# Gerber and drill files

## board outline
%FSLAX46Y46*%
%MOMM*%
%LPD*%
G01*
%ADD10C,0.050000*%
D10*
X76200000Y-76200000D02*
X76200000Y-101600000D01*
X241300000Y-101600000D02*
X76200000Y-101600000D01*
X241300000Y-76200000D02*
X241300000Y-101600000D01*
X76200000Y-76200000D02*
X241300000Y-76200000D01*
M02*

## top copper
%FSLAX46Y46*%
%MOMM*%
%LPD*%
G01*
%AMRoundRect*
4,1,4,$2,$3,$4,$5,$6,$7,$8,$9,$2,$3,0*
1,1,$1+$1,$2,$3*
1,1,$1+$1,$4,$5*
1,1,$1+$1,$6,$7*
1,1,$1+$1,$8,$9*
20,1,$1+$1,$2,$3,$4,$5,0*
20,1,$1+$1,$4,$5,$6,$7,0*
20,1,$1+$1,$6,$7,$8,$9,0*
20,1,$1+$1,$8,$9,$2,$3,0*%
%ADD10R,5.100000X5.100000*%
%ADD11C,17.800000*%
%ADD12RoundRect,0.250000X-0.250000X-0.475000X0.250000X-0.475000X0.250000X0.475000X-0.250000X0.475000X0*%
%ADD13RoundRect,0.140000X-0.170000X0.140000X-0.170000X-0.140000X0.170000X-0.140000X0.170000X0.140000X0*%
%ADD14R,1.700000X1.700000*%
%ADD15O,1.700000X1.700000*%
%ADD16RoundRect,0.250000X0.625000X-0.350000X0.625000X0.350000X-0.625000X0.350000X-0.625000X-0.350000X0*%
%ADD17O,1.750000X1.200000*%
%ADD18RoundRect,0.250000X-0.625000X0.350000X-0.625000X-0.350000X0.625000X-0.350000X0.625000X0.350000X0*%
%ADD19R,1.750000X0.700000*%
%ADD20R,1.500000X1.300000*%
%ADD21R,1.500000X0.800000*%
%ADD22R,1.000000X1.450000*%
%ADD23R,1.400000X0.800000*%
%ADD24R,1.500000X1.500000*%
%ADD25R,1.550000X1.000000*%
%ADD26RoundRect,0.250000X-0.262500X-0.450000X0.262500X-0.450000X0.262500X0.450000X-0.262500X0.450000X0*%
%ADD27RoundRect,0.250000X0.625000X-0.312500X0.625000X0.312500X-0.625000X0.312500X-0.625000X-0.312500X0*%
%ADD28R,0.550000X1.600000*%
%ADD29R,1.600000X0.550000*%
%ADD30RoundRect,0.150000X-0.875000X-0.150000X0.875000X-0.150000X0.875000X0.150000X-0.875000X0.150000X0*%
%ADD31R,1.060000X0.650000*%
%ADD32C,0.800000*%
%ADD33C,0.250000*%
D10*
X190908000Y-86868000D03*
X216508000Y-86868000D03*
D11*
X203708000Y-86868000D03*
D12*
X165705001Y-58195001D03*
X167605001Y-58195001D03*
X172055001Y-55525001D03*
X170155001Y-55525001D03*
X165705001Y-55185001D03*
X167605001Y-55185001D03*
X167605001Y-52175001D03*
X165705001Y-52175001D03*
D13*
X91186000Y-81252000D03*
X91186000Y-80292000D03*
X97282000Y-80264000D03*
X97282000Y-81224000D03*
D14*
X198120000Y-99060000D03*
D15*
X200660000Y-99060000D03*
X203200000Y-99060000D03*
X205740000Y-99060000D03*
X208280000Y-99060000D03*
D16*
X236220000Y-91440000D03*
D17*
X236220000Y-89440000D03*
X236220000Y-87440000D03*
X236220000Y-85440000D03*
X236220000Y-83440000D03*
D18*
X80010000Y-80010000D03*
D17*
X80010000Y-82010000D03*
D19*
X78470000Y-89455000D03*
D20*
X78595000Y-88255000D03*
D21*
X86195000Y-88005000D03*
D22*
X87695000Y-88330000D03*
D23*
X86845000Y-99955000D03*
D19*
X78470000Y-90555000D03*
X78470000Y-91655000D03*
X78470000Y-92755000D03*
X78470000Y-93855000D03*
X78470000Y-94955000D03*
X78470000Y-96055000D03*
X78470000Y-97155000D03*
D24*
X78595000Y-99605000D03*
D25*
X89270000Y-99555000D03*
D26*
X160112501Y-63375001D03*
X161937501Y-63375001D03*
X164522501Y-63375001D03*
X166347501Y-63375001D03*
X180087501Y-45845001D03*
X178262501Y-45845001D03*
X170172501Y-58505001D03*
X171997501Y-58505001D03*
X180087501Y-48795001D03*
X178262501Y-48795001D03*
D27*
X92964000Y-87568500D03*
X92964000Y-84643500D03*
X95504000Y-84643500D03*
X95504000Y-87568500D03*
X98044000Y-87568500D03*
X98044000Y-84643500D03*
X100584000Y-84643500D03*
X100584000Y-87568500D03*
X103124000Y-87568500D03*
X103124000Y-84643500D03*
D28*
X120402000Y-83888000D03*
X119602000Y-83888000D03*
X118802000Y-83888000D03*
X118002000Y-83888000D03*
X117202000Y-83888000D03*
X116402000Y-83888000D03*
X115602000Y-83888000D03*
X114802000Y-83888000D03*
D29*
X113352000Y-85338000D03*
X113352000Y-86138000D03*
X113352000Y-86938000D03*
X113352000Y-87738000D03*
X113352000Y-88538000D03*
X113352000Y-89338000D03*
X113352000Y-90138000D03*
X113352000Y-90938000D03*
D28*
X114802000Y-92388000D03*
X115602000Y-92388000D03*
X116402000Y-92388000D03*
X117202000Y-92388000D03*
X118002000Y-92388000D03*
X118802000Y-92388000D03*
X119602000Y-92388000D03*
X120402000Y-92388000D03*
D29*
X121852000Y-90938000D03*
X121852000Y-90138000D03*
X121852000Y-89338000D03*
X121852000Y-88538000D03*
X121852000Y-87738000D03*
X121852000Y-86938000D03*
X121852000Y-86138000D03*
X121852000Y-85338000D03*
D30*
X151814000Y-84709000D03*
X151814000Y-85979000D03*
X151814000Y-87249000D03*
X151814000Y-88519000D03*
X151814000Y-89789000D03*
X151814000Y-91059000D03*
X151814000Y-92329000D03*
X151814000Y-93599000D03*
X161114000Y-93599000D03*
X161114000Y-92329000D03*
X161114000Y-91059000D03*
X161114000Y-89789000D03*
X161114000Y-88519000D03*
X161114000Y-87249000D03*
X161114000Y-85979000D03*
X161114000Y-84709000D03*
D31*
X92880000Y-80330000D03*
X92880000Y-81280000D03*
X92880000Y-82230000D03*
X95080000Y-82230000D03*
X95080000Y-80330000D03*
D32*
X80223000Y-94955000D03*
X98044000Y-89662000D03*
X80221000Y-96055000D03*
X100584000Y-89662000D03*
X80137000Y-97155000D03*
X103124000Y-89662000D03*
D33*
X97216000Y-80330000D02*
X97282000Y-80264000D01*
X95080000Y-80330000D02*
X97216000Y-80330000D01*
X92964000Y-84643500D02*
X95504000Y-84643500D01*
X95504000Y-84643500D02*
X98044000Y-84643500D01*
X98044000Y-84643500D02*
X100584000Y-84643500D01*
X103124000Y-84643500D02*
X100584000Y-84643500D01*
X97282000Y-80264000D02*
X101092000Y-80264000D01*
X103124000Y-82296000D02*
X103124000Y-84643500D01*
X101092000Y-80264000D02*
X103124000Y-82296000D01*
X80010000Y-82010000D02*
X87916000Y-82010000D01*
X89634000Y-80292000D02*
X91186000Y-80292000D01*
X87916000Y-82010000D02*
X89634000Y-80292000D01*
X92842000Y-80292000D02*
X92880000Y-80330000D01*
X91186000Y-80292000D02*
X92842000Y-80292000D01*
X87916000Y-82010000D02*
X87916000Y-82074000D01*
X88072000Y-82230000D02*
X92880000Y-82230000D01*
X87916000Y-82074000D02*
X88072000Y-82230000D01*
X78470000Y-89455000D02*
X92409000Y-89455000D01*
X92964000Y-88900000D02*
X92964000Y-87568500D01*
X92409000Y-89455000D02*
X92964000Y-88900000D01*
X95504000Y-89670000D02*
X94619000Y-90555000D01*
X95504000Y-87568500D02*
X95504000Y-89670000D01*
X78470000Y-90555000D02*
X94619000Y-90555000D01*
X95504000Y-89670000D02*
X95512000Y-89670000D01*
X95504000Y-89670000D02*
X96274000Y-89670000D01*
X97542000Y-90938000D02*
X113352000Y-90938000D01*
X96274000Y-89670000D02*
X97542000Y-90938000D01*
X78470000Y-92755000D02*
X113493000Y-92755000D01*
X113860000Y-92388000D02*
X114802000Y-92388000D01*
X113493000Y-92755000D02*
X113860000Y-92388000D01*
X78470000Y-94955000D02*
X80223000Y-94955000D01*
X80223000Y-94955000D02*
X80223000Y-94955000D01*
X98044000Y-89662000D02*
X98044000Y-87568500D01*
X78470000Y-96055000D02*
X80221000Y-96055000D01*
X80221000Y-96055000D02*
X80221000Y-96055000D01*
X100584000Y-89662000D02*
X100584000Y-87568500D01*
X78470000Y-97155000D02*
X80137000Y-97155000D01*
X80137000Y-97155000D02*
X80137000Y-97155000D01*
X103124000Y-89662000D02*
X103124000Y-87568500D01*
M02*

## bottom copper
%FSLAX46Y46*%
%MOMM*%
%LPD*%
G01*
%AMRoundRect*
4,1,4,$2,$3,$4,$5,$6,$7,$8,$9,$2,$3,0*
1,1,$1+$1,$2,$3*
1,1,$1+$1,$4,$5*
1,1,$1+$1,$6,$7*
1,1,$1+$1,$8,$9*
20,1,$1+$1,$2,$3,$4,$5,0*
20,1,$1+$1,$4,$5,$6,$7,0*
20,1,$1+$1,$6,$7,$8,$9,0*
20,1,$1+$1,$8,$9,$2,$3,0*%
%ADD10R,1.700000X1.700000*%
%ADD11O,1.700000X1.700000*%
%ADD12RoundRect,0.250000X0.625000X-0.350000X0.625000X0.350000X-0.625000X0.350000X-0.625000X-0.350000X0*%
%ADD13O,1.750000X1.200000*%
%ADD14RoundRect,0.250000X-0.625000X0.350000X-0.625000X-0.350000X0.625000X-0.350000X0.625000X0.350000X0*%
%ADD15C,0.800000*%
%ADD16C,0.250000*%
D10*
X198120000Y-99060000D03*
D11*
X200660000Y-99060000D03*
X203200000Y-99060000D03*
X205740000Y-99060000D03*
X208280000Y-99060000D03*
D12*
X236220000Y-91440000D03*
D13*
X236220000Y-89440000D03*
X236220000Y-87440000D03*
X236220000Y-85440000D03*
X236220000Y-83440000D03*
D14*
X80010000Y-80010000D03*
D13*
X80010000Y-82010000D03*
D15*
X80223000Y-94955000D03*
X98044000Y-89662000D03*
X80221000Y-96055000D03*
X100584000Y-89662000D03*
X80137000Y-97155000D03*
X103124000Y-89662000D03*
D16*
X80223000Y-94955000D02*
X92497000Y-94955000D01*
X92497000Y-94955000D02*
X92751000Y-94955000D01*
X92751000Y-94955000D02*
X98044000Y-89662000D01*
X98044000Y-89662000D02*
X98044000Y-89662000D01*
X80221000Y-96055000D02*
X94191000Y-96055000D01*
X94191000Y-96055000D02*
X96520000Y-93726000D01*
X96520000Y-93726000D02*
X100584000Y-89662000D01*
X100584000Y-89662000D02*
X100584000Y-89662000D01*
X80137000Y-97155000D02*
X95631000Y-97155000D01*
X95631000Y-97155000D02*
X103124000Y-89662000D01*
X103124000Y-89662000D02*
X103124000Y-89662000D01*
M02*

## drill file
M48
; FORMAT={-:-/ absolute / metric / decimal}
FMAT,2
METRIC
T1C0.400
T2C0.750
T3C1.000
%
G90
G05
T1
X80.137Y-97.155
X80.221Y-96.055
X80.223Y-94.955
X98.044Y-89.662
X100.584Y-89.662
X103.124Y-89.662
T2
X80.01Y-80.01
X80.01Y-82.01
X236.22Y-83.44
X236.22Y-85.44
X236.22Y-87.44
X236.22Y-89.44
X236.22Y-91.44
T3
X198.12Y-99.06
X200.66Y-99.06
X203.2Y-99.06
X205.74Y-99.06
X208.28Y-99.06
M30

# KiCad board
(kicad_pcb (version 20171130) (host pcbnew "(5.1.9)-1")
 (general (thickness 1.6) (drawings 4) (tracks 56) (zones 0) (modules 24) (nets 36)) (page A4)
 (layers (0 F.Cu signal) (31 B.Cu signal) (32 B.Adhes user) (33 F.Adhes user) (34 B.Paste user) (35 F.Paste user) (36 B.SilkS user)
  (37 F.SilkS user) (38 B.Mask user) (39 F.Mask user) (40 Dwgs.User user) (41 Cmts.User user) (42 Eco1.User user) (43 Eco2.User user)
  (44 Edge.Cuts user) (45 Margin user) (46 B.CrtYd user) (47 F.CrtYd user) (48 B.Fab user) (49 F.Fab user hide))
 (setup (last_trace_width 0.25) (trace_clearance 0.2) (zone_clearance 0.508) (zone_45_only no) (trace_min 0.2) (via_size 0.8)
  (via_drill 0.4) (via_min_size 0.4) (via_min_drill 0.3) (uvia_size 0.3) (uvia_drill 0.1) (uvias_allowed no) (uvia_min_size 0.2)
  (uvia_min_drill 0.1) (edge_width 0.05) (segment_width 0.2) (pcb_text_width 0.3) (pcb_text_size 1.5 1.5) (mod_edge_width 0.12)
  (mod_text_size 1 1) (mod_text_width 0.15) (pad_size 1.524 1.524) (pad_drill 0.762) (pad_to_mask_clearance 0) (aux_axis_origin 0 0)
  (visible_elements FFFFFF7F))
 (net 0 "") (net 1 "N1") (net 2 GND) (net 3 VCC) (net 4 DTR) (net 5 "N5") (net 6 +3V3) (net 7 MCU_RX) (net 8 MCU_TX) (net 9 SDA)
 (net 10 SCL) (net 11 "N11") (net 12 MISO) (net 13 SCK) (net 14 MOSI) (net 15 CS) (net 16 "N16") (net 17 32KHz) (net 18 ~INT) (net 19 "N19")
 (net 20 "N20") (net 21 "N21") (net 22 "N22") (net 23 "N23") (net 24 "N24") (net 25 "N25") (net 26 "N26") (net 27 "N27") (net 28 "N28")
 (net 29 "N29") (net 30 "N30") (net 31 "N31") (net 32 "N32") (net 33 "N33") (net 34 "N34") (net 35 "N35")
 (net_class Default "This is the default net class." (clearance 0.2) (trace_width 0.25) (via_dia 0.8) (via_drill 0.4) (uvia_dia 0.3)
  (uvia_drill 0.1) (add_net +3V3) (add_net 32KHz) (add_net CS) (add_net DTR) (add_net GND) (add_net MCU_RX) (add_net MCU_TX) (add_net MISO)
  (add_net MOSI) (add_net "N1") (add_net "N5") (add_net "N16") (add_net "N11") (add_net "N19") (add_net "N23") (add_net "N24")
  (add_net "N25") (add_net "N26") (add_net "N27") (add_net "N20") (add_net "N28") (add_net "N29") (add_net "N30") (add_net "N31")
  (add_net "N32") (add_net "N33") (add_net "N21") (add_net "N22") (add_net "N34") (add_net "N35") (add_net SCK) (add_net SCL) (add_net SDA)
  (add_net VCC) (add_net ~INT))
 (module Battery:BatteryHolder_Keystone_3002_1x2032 (layer F.Cu) (at 203.708 86.868 180)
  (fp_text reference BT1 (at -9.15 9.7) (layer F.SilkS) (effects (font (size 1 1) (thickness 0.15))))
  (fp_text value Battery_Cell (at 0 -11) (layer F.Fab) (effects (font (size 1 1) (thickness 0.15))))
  (pad 1 smd rect (at 12.8 0 180) (size 5.1 5.1) (layers F.Cu F.Paste F.Mask) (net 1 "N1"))
  (pad 1 smd rect (at -12.8 0 180) (size 5.1 5.1) (layers F.Cu F.Paste F.Mask) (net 1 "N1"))
  (pad 2 smd circle (at 0 0 180) (size 17.8 17.8) (layers F.Cu F.Mask) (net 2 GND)))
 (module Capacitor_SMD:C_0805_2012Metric (layer F.Cu) (at 166.655001 58.195001)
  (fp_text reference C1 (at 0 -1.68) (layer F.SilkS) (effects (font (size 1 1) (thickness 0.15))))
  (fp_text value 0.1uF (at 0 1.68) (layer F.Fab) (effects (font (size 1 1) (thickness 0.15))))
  (pad 1 smd roundrect (at -0.95 0) (size 1 1.45) (layers F.Cu F.Paste F.Mask) (roundrect_rratio 0.25) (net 2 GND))
  (pad 2 smd roundrect (at 0.95 0) (size 1 1.45) (layers F.Cu F.Paste F.Mask) (roundrect_rratio 0.25) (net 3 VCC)))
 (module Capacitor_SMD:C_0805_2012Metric (layer F.Cu) (at 171.105001 55.525001)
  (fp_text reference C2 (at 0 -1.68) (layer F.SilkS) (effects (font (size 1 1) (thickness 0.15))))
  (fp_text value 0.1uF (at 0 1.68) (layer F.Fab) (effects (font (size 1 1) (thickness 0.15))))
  (pad 2 smd roundrect (at 0.95 0) (size 1 1.45) (layers F.Cu F.Paste F.Mask) (roundrect_rratio 0.25) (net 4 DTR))
  (pad 1 smd roundrect (at -0.95 0) (size 1 1.45) (layers F.Cu F.Paste F.Mask) (roundrect_rratio 0.25) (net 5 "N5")))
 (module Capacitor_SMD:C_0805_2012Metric (layer F.Cu) (at 166.655001 55.185001)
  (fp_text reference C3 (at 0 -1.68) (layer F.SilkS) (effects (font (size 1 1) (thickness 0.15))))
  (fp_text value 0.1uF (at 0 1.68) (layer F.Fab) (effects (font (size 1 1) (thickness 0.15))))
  (pad 1 smd roundrect (at -0.95 0) (size 1 1.45) (layers F.Cu F.Paste F.Mask) (roundrect_rratio 0.25) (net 3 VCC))
  (pad 2 smd roundrect (at 0.95 0) (size 1 1.45) (layers F.Cu F.Paste F.Mask) (roundrect_rratio 0.25) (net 2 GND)))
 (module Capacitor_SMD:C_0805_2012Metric (layer F.Cu) (at 166.655001 52.175001)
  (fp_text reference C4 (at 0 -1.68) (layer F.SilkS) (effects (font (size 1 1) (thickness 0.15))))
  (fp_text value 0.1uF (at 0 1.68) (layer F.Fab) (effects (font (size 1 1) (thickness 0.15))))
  (pad 2 smd roundrect (at 0.95 0) (size 1 1.45) (layers F.Cu F.Paste F.Mask) (roundrect_rratio 0.25) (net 2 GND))
  (pad 1 smd roundrect (at -0.95 0) (size 1 1.45) (layers F.Cu F.Paste F.Mask) (roundrect_rratio 0.25) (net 3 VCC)))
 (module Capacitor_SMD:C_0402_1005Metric (layer F.Cu) (at 91.186 80.772 270)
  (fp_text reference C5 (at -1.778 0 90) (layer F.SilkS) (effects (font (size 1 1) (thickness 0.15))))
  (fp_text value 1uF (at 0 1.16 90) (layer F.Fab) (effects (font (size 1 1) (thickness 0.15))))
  (pad 2 smd roundrect (at 0.48 0 270) (size 0.56 0.62) (layers F.Cu F.Paste F.Mask) (roundrect_rratio 0.25) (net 2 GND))
  (pad 1 smd roundrect (at -0.48 0 270) (size 0.56 0.62) (layers F.Cu F.Paste F.Mask) (roundrect_rratio 0.25) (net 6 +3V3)))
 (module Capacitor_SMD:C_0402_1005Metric (layer F.Cu) (at 97.282 80.744 270)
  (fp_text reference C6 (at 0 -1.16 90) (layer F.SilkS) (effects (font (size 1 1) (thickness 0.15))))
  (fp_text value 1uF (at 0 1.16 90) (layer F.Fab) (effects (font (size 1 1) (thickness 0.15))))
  (pad 1 smd roundrect (at -0.48 0 270) (size 0.56 0.62) (layers F.Cu F.Paste F.Mask) (roundrect_rratio 0.25) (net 3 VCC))
  (pad 2 smd roundrect (at 0.48 0 270) (size 0.56 0.62) (layers F.Cu F.Paste F.Mask) (roundrect_rratio 0.25) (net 2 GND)))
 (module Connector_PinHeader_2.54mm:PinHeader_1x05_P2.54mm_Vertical (layer F.Cu) (at 198.12 99.06 90)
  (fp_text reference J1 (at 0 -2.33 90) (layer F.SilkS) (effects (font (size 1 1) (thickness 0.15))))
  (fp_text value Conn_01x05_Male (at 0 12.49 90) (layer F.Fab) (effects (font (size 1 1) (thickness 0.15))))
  (pad 1 thru_hole rect (at 0 0 90) (size 1.7 1.7) (drill 1) (layers *.Cu *.Mask) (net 2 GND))
  (pad 2 thru_hole oval (at 0 2.54 90) (size 1.7 1.7) (drill 1) (layers *.Cu *.Mask) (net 3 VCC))
  (pad 3 thru_hole oval (at 0 5.08 90) (size 1.7 1.7) (drill 1) (layers *.Cu *.Mask) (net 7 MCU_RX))
  (pad 4 thru_hole oval (at 0 7.62 90) (size 1.7 1.7) (drill 1) (layers *.Cu *.Mask) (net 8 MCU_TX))
  (pad 5 thru_hole oval (at 0 10.16 90) (size 1.7 1.7) (drill 1) (layers *.Cu *.Mask) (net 5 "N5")))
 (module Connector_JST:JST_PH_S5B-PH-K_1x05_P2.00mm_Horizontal (layer F.Cu) (at 236.22 91.44 90)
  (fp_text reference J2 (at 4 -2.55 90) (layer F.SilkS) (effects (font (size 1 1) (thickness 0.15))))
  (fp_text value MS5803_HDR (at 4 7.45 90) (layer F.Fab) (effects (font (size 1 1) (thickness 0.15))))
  (pad 1 thru_hole roundrect (at 0 0 90) (size 1.2 1.75) (drill 0.75) (layers *.Cu *.Mask) (roundrect_rratio 0.208333) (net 2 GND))
  (pad 2 thru_hole oval (at 2 0 90) (size 1.2 1.75) (drill 0.75) (layers *.Cu *.Mask) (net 3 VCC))
  (pad 3 thru_hole oval (at 4 0 90) (size 1.2 1.75) (drill 0.75) (layers *.Cu *.Mask) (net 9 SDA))
  (pad 4 thru_hole oval (at 6 0 90) (size 1.2 1.75) (drill 0.75) (layers *.Cu *.Mask) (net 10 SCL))
  (pad 5 thru_hole oval (at 8 0 90) (size 1.2 1.75) (drill 0.75) (layers *.Cu *.Mask)))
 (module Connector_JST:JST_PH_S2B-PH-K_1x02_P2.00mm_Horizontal (layer F.Cu) (at 80.01 80.01 270)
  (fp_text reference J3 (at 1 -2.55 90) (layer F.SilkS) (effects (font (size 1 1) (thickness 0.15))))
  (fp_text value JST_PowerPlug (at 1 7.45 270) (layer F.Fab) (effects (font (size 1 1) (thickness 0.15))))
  (pad 1 thru_hole roundrect (at 0 0 270) (size 1.2 1.75) (drill 0.75) (layers *.Cu *.Mask) (roundrect_rratio 0.208333) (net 2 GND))
  (pad 2 thru_hole oval (at 2 0 270) (size 1.2 1.75) (drill 0.75) (layers *.Cu *.Mask) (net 6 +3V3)))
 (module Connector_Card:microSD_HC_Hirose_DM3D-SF (layer F.Cu) (at 83.82 93.98 270)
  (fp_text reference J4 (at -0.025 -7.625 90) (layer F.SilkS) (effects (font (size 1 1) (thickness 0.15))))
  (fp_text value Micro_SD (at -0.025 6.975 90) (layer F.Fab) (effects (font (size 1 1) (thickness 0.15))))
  (pad 8 smd rect (at -4.525 5.35 270) (size 0.7 1.75) (layers F.Cu F.Paste F.Mask) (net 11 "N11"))
  (pad 11 smd rect (at -5.725 5.225 270) (size 1.3 1.5) (layers F.Cu F.Paste F.Mask))
  (pad 11 smd rect (at -5.975 -2.375 270) (size 0.8 1.5) (layers F.Cu F.Paste F.Mask))
  (pad 9 smd rect (at -5.65 -3.875 270) (size 1.45 1) (layers F.Cu F.Paste F.Mask) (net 2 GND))
  (pad 11 smd rect (at 5.975 -3.025 270) (size 0.8 1.4) (layers F.Cu F.Paste F.Mask))
  (pad 7 smd rect (at -3.425 5.35 270) (size 0.7 1.75) (layers F.Cu F.Paste F.Mask) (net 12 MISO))
  (pad 6 smd rect (at -2.325 5.35 270) (size 0.7 1.75) (layers F.Cu F.Paste F.Mask) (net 2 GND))
  (pad 5 smd rect (at -1.225 5.35 270) (size 0.7 1.75) (layers F.Cu F.Paste F.Mask) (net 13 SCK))
  (pad 4 smd rect (at -0.125 5.35 270) (size 0.7 1.75) (layers F.Cu F.Paste F.Mask) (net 3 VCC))
  (pad 3 smd rect (at 0.975 5.35 270) (size 0.7 1.75) (layers F.Cu F.Paste F.Mask) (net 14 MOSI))
  (pad 2 smd rect (at 2.075 5.35 270) (size 0.7 1.75) (layers F.Cu F.Paste F.Mask) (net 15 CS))
  (pad 1 smd rect (at 3.175 5.35 270) (size 0.7 1.75) (layers F.Cu F.Paste F.Mask) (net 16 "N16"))
  (pad 11 smd rect (at 5.625 5.225 270) (size 1.5 1.5) (layers F.Cu F.Paste F.Mask))
  (pad 10 smd rect (at 5.575 -5.45 270) (size 1 1.55) (layers F.Cu F.Paste F.Mask)))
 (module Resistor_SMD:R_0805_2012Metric (layer F.Cu) (at 161.025001 63.375001)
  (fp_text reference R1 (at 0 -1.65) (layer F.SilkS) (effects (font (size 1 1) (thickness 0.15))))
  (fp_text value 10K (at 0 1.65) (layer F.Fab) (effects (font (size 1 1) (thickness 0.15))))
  (pad 1 smd roundrect (at -0.9125 0) (size 1.025 1.4) (layers F.Cu F.Paste F.Mask) (roundrect_rratio 0.243902) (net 3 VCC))
  (pad 2 smd roundrect (at 0.9125 0) (size 1.025 1.4) (layers F.Cu F.Paste F.Mask) (roundrect_rratio 0.243902) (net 4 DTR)))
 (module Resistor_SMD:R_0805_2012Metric (layer F.Cu) (at 165.435001 63.375001)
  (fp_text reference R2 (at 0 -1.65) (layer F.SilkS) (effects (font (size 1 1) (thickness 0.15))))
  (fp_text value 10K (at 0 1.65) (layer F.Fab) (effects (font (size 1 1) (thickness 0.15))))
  (pad 1 smd roundrect (at -0.9125 0) (size 1.025 1.4) (layers F.Cu F.Paste F.Mask) (roundrect_rratio 0.243902) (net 3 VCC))
  (pad 2 smd roundrect (at 0.9125 0) (size 1.025 1.4) (layers F.Cu F.Paste F.Mask) (roundrect_rratio 0.243902) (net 10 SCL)))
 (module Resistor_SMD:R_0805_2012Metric (layer F.Cu) (at 179.175001 45.845001)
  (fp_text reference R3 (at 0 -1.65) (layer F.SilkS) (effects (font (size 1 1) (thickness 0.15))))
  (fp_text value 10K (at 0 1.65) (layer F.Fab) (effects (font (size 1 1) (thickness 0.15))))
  (pad 2 smd roundrect (at 0.9125 0) (size 1.025 1.4) (layers F.Cu F.Paste F.Mask) (roundrect_rratio 0.243902) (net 9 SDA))
  (pad 1 smd roundrect (at -0.9125 0) (size 1.025 1.4) (layers F.Cu F.Paste F.Mask) (roundrect_rratio 0.243902) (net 3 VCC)))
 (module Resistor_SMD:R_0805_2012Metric (layer F.Cu) (at 171.085001 58.505001)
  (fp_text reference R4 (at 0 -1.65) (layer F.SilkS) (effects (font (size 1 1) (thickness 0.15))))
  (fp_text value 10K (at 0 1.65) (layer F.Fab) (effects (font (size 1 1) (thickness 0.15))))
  (pad 1 smd roundrect (at -0.9125 0) (size 1.025 1.4) (layers F.Cu F.Paste F.Mask) (roundrect_rratio 0.243902) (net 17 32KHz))
  (pad 2 smd roundrect (at 0.9125 0) (size 1.025 1.4) (layers F.Cu F.Paste F.Mask) (roundrect_rratio 0.243902) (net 3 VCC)))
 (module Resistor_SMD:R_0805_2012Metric (layer F.Cu) (at 179.175001 48.795001)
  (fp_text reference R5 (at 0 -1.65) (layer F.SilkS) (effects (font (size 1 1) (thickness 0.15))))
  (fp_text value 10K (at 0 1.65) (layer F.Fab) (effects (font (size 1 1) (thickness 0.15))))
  (pad 2 smd roundrect (at 0.9125 0) (size 1.025 1.4) (layers F.Cu F.Paste F.Mask) (roundrect_rratio 0.243902) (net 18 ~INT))
  (pad 1 smd roundrect (at -0.9125 0) (size 1.025 1.4) (layers F.Cu F.Paste F.Mask) (roundrect_rratio 0.243902) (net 3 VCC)))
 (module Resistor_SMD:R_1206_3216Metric (layer F.Cu) (at 92.964 86.106 90)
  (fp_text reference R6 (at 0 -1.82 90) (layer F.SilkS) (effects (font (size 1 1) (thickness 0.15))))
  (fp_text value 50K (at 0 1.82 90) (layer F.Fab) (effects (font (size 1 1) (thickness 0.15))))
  (pad 1 smd roundrect (at -1.4625 0 90) (size 1.125 1.75) (layers F.Cu F.Paste F.Mask) (roundrect_rratio 0.222222) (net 11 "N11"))
  (pad 2 smd roundrect (at 1.4625 0 90) (size 1.125 1.75) (layers F.Cu F.Paste F.Mask) (roundrect_rratio 0.222222) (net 3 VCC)))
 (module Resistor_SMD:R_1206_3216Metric (layer F.Cu) (at 95.504 86.106 90)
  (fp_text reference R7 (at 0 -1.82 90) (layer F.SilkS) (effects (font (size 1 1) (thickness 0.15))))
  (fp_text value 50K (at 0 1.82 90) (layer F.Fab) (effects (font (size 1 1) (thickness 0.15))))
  (pad 2 smd roundrect (at 1.4625 0 90) (size 1.125 1.75) (layers F.Cu F.Paste F.Mask) (roundrect_rratio 0.222222) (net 3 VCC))
  (pad 1 smd roundrect (at -1.4625 0 90) (size 1.125 1.75) (layers F.Cu F.Paste F.Mask) (roundrect_rratio 0.222222) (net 12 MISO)))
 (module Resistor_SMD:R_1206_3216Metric (layer F.Cu) (at 98.044 86.106 90)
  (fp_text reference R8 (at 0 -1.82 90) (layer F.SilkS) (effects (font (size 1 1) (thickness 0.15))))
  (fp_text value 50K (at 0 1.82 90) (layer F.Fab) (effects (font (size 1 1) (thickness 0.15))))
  (pad 1 smd roundrect (at -1.4625 0 90) (size 1.125 1.75) (layers F.Cu F.Paste F.Mask) (roundrect_rratio 0.222222) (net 14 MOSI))
  (pad 2 smd roundrect (at 1.4625 0 90) (size 1.125 1.75) (layers F.Cu F.Paste F.Mask) (roundrect_rratio 0.222222) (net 3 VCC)))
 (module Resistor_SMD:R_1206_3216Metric (layer F.Cu) (at 100.584 86.106 90)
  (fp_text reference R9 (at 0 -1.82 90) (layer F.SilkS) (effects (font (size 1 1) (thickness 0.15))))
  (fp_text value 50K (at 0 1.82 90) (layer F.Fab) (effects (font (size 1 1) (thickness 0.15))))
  (pad 2 smd roundrect (at 1.4625 0 90) (size 1.125 1.75) (layers F.Cu F.Paste F.Mask) (roundrect_rratio 0.222222) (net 3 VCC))
  (pad 1 smd roundrect (at -1.4625 0 90) (size 1.125 1.75) (layers F.Cu F.Paste F.Mask) (roundrect_rratio 0.222222) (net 15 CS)))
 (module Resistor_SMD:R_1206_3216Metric (layer F.Cu) (at 103.124 86.106 90)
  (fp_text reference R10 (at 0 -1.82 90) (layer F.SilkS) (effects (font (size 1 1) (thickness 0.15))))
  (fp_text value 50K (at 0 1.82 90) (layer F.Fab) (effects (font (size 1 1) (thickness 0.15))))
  (pad 1 smd roundrect (at -1.4625 0 90) (size 1.125 1.75) (layers F.Cu F.Paste F.Mask) (roundrect_rratio 0.222222) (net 16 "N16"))
  (pad 2 smd roundrect (at 1.4625 0 90) (size 1.125 1.75) (layers F.Cu F.Paste F.Mask) (roundrect_rratio 0.222222) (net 3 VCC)))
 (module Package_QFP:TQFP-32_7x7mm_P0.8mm (layer F.Cu) (at 117.602 88.138 270)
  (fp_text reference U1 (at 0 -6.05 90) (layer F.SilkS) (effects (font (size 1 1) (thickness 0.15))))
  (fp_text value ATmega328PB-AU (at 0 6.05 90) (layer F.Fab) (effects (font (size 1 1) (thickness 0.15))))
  (pad 1 smd rect (at -4.25 -2.8 270) (size 1.6 0.55) (layers F.Cu F.Paste F.Mask) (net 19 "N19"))
  (pad 2 smd rect (at -4.25 -2 270) (size 1.6 0.55) (layers F.Cu F.Paste F.Mask) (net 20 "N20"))
  (pad 3 smd rect (at -4.25 -1.2 270) (size 1.6 0.55) (layers F.Cu F.Paste F.Mask) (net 2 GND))
  (pad 4 smd rect (at -4.25 -0.4 270) (size 1.6 0.55) (layers F.Cu F.Paste F.Mask) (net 3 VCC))
  (pad 5 smd rect (at -4.25 0.4 270) (size 1.6 0.55) (layers F.Cu F.Paste F.Mask) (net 2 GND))
  (pad 6 smd rect (at -4.25 1.2 270) (size 1.6 0.55) (layers F.Cu F.Paste F.Mask) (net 3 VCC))
  (pad 7 smd rect (at -4.25 2 270) (size 1.6 0.55) (layers F.Cu F.Paste F.Mask) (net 17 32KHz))
  (pad 8 smd rect (at -4.25 2.8 270) (size 1.6 0.55) (layers F.Cu F.Paste F.Mask) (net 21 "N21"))
  (pad 9 smd rect (at -2.8 4.25) (size 1.6 0.55) (layers F.Cu F.Paste F.Mask) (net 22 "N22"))
  (pad 10 smd rect (at -2 4.25) (size 1.6 0.55) (layers F.Cu F.Paste F.Mask) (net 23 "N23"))
  (pad 11 smd rect (at -1.2 4.25) (size 1.6 0.55) (layers F.Cu F.Paste F.Mask) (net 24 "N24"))
  (pad 12 smd rect (at -0.4 4.25) (size 1.6 0.55) (layers F.Cu F.Paste F.Mask) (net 15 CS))
  (pad 13 smd rect (at 0.4 4.25) (size 1.6 0.55) (layers F.Cu F.Paste F.Mask) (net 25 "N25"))
  (pad 14 smd rect (at 1.2 4.25) (size 1.6 0.55) (layers F.Cu F.Paste F.Mask) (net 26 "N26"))
  (pad 15 smd rect (at 2 4.25) (size 1.6 0.55) (layers F.Cu F.Paste F.Mask) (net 14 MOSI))
  (pad 16 smd rect (at 2.8 4.25) (size 1.6 0.55) (layers F.Cu F.Paste F.Mask) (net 12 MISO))
  (pad 17 smd rect (at 4.25 2.8 270) (size 1.6 0.55) (layers F.Cu F.Paste F.Mask) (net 13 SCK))
  (pad 18 smd rect (at 4.25 2 270) (size 1.6 0.55) (layers F.Cu F.Paste F.Mask) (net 3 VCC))
  (pad 19 smd rect (at 4.25 1.2 270) (size 1.6 0.55) (layers F.Cu F.Paste F.Mask) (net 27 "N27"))
  (pad 20 smd rect (at 4.25 0.4 270) (size 1.6 0.55) (layers F.Cu F.Paste F.Mask) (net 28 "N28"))
  (pad 21 smd rect (at 4.25 -0.4 270) (size 1.6 0.55) (layers F.Cu F.Paste F.Mask) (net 2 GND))
  (pad 22 smd rect (at 4.25 -1.2 270) (size 1.6 0.55) (layers F.Cu F.Paste F.Mask) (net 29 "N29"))
  (pad 23 smd rect (at 4.25 -2 270) (size 1.6 0.55) (layers F.Cu F.Paste F.Mask) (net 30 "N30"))
  (pad 24 smd rect (at 4.25 -2.8 270) (size 1.6 0.55) (layers F.Cu F.Paste F.Mask) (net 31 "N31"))
  (pad 25 smd rect (at 2.8 -4.25) (size 1.6 0.55) (layers F.Cu F.Paste F.Mask) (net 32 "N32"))
  (pad 26 smd rect (at 2 -4.25) (size 1.6 0.55) (layers F.Cu F.Paste F.Mask) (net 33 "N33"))
  (pad 27 smd rect (at 1.2 -4.25) (size 1.6 0.55) (layers F.Cu F.Paste F.Mask) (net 9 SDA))
  (pad 28 smd rect (at 0.4 -4.25) (size 1.6 0.55) (layers F.Cu F.Paste F.Mask) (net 10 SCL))
  (pad 29 smd rect (at -0.4 -4.25) (size 1.6 0.55) (layers F.Cu F.Paste F.Mask) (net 4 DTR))
  (pad 30 smd rect (at -1.2 -4.25) (size 1.6 0.55) (layers F.Cu F.Paste F.Mask) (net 7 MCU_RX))
  (pad 31 smd rect (at -2 -4.25) (size 1.6 0.55) (layers F.Cu F.Paste F.Mask) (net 8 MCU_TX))
  (pad 32 smd rect (at -2.8 -4.25) (size 1.6 0.55) (layers F.Cu F.Paste F.Mask) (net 18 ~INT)))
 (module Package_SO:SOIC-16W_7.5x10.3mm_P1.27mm (layer F.Cu) (at 156.464 89.154)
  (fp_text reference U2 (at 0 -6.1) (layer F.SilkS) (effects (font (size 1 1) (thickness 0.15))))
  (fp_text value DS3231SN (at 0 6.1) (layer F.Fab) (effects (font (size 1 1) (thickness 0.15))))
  (pad 1 smd roundrect (at -4.65 -4.445) (size 2.05 0.6) (layers F.Cu F.Paste F.Mask) (roundrect_rratio 0.25) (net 17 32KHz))
  (pad 2 smd roundrect (at -4.65 -3.175) (size 2.05 0.6) (layers F.Cu F.Paste F.Mask) (roundrect_rratio 0.25) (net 3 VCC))
  (pad 3 smd roundrect (at -4.65 -1.905) (size 2.05 0.6) (layers F.Cu F.Paste F.Mask) (roundrect_rratio 0.25) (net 18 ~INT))
  (pad 4 smd roundrect (at -4.65 -0.635) (size 2.05 0.6) (layers F.Cu F.Paste F.Mask) (roundrect_rratio 0.25) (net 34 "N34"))
  (pad 5 smd roundrect (at -4.65 0.635) (size 2.05 0.6) (layers F.Cu F.Paste F.Mask) (roundrect_rratio 0.25) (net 2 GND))
  (pad 6 smd roundrect (at -4.65 1.905) (size 2.05 0.6) (layers F.Cu F.Paste F.Mask) (roundrect_rratio 0.25) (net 2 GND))
  (pad 7 smd roundrect (at -4.65 3.175) (size 2.05 0.6) (layers F.Cu F.Paste F.Mask) (roundrect_rratio 0.25) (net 2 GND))
  (pad 8 smd roundrect (at -4.65 4.445) (size 2.05 0.6) (layers F.Cu F.Paste F.Mask) (roundrect_rratio 0.25) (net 2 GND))
  (pad 9 smd roundrect (at 4.65 4.445) (size 2.05 0.6) (layers F.Cu F.Paste F.Mask) (roundrect_rratio 0.25) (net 2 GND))
  (pad 10 smd roundrect (at 4.65 3.175) (size 2.05 0.6) (layers F.Cu F.Paste F.Mask) (roundrect_rratio 0.25) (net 2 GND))
  (pad 11 smd roundrect (at 4.65 1.905) (size 2.05 0.6) (layers F.Cu F.Paste F.Mask) (roundrect_rratio 0.25) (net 2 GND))
  (pad 12 smd roundrect (at 4.65 0.635) (size 2.05 0.6) (layers F.Cu F.Paste F.Mask) (roundrect_rratio 0.25) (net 2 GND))
  (pad 13 smd roundrect (at 4.65 -0.635) (size 2.05 0.6) (layers F.Cu F.Paste F.Mask) (roundrect_rratio 0.25) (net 2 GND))
  (pad 14 smd roundrect (at 4.65 -1.905) (size 2.05 0.6) (layers F.Cu F.Paste F.Mask) (roundrect_rratio 0.25) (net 1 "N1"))
  (pad 15 smd roundrect (at 4.65 -3.175) (size 2.05 0.6) (layers F.Cu F.Paste F.Mask) (roundrect_rratio 0.25) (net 9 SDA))
  (pad 16 smd roundrect (at 4.65 -4.445) (size 2.05 0.6) (layers F.Cu F.Paste F.Mask) (roundrect_rratio 0.25) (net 10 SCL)))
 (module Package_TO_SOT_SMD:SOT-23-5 (layer F.Cu) (at 93.98 81.28)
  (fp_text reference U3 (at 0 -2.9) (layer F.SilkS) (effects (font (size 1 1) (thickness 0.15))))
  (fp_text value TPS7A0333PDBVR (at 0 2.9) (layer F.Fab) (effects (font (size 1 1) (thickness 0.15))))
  (pad 1 smd rect (at -1.1 -0.95) (size 1.06 0.65) (layers F.Cu F.Paste F.Mask) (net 6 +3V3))
  (pad 2 smd rect (at -1.1 0) (size 1.06 0.65) (layers F.Cu F.Paste F.Mask) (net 2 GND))
  (pad 3 smd rect (at -1.1 0.95) (size 1.06 0.65) (layers F.Cu F.Paste F.Mask) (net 6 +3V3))
  (pad 4 smd rect (at 1.1 0.95) (size 1.06 0.65) (layers F.Cu F.Paste F.Mask) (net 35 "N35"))
  (pad 5 smd rect (at 1.1 -0.95) (size 1.06 0.65) (layers F.Cu F.Paste F.Mask) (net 3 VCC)))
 (gr_line (start 76.2 76.2) (end 76.2 101.6) (layer Edge.Cuts) (width 0.05))
 (gr_line (start 241.3 101.6) (end 76.2 101.6) (layer Edge.Cuts) (width 0.05))
 (gr_line (start 241.3 76.2) (end 241.3 101.6) (layer Edge.Cuts) (width 0.05))
 (gr_line (start 76.2 76.2) (end 241.3 76.2) (layer Edge.Cuts) (width 0.05))
 (segment (start 97.216 80.33) (end 97.282 80.264) (width 0.25) (layer F.Cu) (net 3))
 (segment (start 95.08 80.33) (end 97.216 80.33) (width 0.25) (layer F.Cu) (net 3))
 (segment (start 92.964 84.6435) (end 95.504 84.6435) (width 0.25) (layer F.Cu) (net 3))
 (segment (start 95.504 84.6435) (end 98.044 84.6435) (width 0.25) (layer F.Cu) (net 3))
 (segment (start 98.044 84.6435) (end 100.584 84.6435) (width 0.25) (layer F.Cu) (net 3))
 (segment (start 103.124 84.6435) (end 100.584 84.6435) (width 0.25) (layer F.Cu) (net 3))
 (segment (start 97.282 80.264) (end 101.092 80.264) (width 0.25) (layer F.Cu) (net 3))
 (segment (start 103.124 82.296) (end 103.124 84.6435) (width 0.25) (layer F.Cu) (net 3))
 (segment (start 101.092 80.264) (end 103.124 82.296) (width 0.25) (layer F.Cu) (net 3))
 (segment (start 80.01 82.01) (end 87.916 82.01) (width 0.25) (layer F.Cu) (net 6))
 (segment (start 89.634 80.292) (end 91.186 80.292) (width 0.25) (layer F.Cu) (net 6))
 (segment (start 87.916 82.01) (end 89.634 80.292) (width 0.25) (layer F.Cu) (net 6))
 (segment (start 92.842 80.292) (end 92.88 80.33) (width 0.25) (layer F.Cu) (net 6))
 (segment (start 91.186 80.292) (end 92.842 80.292) (width 0.25) (layer F.Cu) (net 6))
 (segment (start 87.916 82.01) (end 87.916 82.074) (width 0.25) (layer F.Cu) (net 6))
 (segment (start 88.072 82.23) (end 92.88 82.23) (width 0.25) (layer F.Cu) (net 6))
 (segment (start 87.916 82.074) (end 88.072 82.23) (width 0.25) (layer F.Cu) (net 6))
 (segment (start 78.47 89.455) (end 92.409 89.455) (width 0.25) (layer F.Cu) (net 11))
 (segment (start 92.964 88.9) (end 92.964 87.5685) (width 0.25) (layer F.Cu) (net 11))
 (segment (start 92.409 89.455) (end 92.964 88.9) (width 0.25) (layer F.Cu) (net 11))
 (segment (start 95.504 89.67) (end 94.619 90.555) (width 0.25) (layer F.Cu) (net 12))
 (segment (start 95.504 87.5685) (end 95.504 89.67) (width 0.25) (layer F.Cu) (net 12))
 (segment (start 78.47 90.555) (end 94.619 90.555) (width 0.25) (layer F.Cu) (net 12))
 (segment (start 95.504 89.67) (end 95.512 89.67) (width 0.25) (layer F.Cu) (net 12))
 (segment (start 95.504 89.67) (end 96.274 89.67) (width 0.25) (layer F.Cu) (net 12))
 (segment (start 97.542 90.938) (end 113.352 90.938) (width 0.25) (layer F.Cu) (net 12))
 (segment (start 96.274 89.67) (end 97.542 90.938) (width 0.25) (layer F.Cu) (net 12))
 (segment (start 78.47 92.755) (end 113.493 92.755) (width 0.25) (layer F.Cu) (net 13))
 (segment (start 113.86 92.388) (end 114.802 92.388) (width 0.25) (layer F.Cu) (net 13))
 (segment (start 113.493 92.755) (end 113.86 92.388) (width 0.25) (layer F.Cu) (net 13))
 (segment (start 78.47 94.955) (end 80.223 94.955) (width 0.25) (layer F.Cu) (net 14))
 (segment (start 80.223 94.955) (end 80.223 94.955) (width 0.25) (layer F.Cu) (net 14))
 (via (at 80.223 94.955) (size 0.8) (drill 0.4) (layers F.Cu B.Cu) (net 14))
 (segment (start 80.223 94.955) (end 92.497 94.955) (width 0.25) (layer B.Cu) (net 14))
 (segment (start 92.497 94.955) (end 92.751 94.955) (width 0.25) (layer B.Cu) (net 14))
 (segment (start 92.751 94.955) (end 98.044 89.662) (width 0.25) (layer B.Cu) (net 14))
 (segment (start 98.044 89.662) (end 98.044 89.662) (width 0.25) (layer B.Cu) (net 14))
 (via (at 98.044 89.662) (size 0.8) (drill 0.4) (layers F.Cu B.Cu) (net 14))
 (segment (start 98.044 89.662) (end 98.044 87.5685) (width 0.25) (layer F.Cu) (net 14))
 (segment (start 78.47 96.055) (end 80.221 96.055) (width 0.25) (layer F.Cu) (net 15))
 (segment (start 80.221 96.055) (end 80.221 96.055) (width 0.25) (layer F.Cu) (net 15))
 (via (at 80.221 96.055) (size 0.8) (drill 0.4) (layers F.Cu B.Cu) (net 15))
 (segment (start 80.221 96.055) (end 94.191 96.055) (width 0.25) (layer B.Cu) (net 15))
 (segment (start 94.191 96.055) (end 96.52 93.726) (width 0.25) (layer B.Cu) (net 15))
 (segment (start 96.52 93.726) (end 100.584 89.662) (width 0.25) (layer B.Cu) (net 15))
 (segment (start 100.584 89.662) (end 100.584 89.662) (width 0.25) (layer B.Cu) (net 15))
 (via (at 100.584 89.662) (size 0.8) (drill 0.4) (layers F.Cu B.Cu) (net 15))
 (segment (start 100.584 89.662) (end 100.584 87.5685) (width 0.25) (layer F.Cu) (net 15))
 (segment (start 78.47 97.155) (end 80.137 97.155) (width 0.25) (layer F.Cu) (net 16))
 (segment (start 80.137 97.155) (end 80.137 97.155) (width 0.25) (layer F.Cu) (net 16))
 (via (at 80.137 97.155) (size 0.8) (drill 0.4) (layers F.Cu B.Cu) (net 16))
 (segment (start 80.137 97.155) (end 95.631 97.155) (width 0.25) (layer B.Cu) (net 16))
 (segment (start 95.631 97.155) (end 103.124 89.662) (width 0.25) (layer B.Cu) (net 16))
 (segment (start 103.124 89.662) (end 103.124 89.662) (width 0.25) (layer B.Cu) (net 16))
 (via (at 103.124 89.662) (size 0.8) (drill 0.4) (layers F.Cu B.Cu) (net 16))
 (segment (start 103.124 89.662) (end 103.124 87.5685) (width 0.25) (layer F.Cu) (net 16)))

